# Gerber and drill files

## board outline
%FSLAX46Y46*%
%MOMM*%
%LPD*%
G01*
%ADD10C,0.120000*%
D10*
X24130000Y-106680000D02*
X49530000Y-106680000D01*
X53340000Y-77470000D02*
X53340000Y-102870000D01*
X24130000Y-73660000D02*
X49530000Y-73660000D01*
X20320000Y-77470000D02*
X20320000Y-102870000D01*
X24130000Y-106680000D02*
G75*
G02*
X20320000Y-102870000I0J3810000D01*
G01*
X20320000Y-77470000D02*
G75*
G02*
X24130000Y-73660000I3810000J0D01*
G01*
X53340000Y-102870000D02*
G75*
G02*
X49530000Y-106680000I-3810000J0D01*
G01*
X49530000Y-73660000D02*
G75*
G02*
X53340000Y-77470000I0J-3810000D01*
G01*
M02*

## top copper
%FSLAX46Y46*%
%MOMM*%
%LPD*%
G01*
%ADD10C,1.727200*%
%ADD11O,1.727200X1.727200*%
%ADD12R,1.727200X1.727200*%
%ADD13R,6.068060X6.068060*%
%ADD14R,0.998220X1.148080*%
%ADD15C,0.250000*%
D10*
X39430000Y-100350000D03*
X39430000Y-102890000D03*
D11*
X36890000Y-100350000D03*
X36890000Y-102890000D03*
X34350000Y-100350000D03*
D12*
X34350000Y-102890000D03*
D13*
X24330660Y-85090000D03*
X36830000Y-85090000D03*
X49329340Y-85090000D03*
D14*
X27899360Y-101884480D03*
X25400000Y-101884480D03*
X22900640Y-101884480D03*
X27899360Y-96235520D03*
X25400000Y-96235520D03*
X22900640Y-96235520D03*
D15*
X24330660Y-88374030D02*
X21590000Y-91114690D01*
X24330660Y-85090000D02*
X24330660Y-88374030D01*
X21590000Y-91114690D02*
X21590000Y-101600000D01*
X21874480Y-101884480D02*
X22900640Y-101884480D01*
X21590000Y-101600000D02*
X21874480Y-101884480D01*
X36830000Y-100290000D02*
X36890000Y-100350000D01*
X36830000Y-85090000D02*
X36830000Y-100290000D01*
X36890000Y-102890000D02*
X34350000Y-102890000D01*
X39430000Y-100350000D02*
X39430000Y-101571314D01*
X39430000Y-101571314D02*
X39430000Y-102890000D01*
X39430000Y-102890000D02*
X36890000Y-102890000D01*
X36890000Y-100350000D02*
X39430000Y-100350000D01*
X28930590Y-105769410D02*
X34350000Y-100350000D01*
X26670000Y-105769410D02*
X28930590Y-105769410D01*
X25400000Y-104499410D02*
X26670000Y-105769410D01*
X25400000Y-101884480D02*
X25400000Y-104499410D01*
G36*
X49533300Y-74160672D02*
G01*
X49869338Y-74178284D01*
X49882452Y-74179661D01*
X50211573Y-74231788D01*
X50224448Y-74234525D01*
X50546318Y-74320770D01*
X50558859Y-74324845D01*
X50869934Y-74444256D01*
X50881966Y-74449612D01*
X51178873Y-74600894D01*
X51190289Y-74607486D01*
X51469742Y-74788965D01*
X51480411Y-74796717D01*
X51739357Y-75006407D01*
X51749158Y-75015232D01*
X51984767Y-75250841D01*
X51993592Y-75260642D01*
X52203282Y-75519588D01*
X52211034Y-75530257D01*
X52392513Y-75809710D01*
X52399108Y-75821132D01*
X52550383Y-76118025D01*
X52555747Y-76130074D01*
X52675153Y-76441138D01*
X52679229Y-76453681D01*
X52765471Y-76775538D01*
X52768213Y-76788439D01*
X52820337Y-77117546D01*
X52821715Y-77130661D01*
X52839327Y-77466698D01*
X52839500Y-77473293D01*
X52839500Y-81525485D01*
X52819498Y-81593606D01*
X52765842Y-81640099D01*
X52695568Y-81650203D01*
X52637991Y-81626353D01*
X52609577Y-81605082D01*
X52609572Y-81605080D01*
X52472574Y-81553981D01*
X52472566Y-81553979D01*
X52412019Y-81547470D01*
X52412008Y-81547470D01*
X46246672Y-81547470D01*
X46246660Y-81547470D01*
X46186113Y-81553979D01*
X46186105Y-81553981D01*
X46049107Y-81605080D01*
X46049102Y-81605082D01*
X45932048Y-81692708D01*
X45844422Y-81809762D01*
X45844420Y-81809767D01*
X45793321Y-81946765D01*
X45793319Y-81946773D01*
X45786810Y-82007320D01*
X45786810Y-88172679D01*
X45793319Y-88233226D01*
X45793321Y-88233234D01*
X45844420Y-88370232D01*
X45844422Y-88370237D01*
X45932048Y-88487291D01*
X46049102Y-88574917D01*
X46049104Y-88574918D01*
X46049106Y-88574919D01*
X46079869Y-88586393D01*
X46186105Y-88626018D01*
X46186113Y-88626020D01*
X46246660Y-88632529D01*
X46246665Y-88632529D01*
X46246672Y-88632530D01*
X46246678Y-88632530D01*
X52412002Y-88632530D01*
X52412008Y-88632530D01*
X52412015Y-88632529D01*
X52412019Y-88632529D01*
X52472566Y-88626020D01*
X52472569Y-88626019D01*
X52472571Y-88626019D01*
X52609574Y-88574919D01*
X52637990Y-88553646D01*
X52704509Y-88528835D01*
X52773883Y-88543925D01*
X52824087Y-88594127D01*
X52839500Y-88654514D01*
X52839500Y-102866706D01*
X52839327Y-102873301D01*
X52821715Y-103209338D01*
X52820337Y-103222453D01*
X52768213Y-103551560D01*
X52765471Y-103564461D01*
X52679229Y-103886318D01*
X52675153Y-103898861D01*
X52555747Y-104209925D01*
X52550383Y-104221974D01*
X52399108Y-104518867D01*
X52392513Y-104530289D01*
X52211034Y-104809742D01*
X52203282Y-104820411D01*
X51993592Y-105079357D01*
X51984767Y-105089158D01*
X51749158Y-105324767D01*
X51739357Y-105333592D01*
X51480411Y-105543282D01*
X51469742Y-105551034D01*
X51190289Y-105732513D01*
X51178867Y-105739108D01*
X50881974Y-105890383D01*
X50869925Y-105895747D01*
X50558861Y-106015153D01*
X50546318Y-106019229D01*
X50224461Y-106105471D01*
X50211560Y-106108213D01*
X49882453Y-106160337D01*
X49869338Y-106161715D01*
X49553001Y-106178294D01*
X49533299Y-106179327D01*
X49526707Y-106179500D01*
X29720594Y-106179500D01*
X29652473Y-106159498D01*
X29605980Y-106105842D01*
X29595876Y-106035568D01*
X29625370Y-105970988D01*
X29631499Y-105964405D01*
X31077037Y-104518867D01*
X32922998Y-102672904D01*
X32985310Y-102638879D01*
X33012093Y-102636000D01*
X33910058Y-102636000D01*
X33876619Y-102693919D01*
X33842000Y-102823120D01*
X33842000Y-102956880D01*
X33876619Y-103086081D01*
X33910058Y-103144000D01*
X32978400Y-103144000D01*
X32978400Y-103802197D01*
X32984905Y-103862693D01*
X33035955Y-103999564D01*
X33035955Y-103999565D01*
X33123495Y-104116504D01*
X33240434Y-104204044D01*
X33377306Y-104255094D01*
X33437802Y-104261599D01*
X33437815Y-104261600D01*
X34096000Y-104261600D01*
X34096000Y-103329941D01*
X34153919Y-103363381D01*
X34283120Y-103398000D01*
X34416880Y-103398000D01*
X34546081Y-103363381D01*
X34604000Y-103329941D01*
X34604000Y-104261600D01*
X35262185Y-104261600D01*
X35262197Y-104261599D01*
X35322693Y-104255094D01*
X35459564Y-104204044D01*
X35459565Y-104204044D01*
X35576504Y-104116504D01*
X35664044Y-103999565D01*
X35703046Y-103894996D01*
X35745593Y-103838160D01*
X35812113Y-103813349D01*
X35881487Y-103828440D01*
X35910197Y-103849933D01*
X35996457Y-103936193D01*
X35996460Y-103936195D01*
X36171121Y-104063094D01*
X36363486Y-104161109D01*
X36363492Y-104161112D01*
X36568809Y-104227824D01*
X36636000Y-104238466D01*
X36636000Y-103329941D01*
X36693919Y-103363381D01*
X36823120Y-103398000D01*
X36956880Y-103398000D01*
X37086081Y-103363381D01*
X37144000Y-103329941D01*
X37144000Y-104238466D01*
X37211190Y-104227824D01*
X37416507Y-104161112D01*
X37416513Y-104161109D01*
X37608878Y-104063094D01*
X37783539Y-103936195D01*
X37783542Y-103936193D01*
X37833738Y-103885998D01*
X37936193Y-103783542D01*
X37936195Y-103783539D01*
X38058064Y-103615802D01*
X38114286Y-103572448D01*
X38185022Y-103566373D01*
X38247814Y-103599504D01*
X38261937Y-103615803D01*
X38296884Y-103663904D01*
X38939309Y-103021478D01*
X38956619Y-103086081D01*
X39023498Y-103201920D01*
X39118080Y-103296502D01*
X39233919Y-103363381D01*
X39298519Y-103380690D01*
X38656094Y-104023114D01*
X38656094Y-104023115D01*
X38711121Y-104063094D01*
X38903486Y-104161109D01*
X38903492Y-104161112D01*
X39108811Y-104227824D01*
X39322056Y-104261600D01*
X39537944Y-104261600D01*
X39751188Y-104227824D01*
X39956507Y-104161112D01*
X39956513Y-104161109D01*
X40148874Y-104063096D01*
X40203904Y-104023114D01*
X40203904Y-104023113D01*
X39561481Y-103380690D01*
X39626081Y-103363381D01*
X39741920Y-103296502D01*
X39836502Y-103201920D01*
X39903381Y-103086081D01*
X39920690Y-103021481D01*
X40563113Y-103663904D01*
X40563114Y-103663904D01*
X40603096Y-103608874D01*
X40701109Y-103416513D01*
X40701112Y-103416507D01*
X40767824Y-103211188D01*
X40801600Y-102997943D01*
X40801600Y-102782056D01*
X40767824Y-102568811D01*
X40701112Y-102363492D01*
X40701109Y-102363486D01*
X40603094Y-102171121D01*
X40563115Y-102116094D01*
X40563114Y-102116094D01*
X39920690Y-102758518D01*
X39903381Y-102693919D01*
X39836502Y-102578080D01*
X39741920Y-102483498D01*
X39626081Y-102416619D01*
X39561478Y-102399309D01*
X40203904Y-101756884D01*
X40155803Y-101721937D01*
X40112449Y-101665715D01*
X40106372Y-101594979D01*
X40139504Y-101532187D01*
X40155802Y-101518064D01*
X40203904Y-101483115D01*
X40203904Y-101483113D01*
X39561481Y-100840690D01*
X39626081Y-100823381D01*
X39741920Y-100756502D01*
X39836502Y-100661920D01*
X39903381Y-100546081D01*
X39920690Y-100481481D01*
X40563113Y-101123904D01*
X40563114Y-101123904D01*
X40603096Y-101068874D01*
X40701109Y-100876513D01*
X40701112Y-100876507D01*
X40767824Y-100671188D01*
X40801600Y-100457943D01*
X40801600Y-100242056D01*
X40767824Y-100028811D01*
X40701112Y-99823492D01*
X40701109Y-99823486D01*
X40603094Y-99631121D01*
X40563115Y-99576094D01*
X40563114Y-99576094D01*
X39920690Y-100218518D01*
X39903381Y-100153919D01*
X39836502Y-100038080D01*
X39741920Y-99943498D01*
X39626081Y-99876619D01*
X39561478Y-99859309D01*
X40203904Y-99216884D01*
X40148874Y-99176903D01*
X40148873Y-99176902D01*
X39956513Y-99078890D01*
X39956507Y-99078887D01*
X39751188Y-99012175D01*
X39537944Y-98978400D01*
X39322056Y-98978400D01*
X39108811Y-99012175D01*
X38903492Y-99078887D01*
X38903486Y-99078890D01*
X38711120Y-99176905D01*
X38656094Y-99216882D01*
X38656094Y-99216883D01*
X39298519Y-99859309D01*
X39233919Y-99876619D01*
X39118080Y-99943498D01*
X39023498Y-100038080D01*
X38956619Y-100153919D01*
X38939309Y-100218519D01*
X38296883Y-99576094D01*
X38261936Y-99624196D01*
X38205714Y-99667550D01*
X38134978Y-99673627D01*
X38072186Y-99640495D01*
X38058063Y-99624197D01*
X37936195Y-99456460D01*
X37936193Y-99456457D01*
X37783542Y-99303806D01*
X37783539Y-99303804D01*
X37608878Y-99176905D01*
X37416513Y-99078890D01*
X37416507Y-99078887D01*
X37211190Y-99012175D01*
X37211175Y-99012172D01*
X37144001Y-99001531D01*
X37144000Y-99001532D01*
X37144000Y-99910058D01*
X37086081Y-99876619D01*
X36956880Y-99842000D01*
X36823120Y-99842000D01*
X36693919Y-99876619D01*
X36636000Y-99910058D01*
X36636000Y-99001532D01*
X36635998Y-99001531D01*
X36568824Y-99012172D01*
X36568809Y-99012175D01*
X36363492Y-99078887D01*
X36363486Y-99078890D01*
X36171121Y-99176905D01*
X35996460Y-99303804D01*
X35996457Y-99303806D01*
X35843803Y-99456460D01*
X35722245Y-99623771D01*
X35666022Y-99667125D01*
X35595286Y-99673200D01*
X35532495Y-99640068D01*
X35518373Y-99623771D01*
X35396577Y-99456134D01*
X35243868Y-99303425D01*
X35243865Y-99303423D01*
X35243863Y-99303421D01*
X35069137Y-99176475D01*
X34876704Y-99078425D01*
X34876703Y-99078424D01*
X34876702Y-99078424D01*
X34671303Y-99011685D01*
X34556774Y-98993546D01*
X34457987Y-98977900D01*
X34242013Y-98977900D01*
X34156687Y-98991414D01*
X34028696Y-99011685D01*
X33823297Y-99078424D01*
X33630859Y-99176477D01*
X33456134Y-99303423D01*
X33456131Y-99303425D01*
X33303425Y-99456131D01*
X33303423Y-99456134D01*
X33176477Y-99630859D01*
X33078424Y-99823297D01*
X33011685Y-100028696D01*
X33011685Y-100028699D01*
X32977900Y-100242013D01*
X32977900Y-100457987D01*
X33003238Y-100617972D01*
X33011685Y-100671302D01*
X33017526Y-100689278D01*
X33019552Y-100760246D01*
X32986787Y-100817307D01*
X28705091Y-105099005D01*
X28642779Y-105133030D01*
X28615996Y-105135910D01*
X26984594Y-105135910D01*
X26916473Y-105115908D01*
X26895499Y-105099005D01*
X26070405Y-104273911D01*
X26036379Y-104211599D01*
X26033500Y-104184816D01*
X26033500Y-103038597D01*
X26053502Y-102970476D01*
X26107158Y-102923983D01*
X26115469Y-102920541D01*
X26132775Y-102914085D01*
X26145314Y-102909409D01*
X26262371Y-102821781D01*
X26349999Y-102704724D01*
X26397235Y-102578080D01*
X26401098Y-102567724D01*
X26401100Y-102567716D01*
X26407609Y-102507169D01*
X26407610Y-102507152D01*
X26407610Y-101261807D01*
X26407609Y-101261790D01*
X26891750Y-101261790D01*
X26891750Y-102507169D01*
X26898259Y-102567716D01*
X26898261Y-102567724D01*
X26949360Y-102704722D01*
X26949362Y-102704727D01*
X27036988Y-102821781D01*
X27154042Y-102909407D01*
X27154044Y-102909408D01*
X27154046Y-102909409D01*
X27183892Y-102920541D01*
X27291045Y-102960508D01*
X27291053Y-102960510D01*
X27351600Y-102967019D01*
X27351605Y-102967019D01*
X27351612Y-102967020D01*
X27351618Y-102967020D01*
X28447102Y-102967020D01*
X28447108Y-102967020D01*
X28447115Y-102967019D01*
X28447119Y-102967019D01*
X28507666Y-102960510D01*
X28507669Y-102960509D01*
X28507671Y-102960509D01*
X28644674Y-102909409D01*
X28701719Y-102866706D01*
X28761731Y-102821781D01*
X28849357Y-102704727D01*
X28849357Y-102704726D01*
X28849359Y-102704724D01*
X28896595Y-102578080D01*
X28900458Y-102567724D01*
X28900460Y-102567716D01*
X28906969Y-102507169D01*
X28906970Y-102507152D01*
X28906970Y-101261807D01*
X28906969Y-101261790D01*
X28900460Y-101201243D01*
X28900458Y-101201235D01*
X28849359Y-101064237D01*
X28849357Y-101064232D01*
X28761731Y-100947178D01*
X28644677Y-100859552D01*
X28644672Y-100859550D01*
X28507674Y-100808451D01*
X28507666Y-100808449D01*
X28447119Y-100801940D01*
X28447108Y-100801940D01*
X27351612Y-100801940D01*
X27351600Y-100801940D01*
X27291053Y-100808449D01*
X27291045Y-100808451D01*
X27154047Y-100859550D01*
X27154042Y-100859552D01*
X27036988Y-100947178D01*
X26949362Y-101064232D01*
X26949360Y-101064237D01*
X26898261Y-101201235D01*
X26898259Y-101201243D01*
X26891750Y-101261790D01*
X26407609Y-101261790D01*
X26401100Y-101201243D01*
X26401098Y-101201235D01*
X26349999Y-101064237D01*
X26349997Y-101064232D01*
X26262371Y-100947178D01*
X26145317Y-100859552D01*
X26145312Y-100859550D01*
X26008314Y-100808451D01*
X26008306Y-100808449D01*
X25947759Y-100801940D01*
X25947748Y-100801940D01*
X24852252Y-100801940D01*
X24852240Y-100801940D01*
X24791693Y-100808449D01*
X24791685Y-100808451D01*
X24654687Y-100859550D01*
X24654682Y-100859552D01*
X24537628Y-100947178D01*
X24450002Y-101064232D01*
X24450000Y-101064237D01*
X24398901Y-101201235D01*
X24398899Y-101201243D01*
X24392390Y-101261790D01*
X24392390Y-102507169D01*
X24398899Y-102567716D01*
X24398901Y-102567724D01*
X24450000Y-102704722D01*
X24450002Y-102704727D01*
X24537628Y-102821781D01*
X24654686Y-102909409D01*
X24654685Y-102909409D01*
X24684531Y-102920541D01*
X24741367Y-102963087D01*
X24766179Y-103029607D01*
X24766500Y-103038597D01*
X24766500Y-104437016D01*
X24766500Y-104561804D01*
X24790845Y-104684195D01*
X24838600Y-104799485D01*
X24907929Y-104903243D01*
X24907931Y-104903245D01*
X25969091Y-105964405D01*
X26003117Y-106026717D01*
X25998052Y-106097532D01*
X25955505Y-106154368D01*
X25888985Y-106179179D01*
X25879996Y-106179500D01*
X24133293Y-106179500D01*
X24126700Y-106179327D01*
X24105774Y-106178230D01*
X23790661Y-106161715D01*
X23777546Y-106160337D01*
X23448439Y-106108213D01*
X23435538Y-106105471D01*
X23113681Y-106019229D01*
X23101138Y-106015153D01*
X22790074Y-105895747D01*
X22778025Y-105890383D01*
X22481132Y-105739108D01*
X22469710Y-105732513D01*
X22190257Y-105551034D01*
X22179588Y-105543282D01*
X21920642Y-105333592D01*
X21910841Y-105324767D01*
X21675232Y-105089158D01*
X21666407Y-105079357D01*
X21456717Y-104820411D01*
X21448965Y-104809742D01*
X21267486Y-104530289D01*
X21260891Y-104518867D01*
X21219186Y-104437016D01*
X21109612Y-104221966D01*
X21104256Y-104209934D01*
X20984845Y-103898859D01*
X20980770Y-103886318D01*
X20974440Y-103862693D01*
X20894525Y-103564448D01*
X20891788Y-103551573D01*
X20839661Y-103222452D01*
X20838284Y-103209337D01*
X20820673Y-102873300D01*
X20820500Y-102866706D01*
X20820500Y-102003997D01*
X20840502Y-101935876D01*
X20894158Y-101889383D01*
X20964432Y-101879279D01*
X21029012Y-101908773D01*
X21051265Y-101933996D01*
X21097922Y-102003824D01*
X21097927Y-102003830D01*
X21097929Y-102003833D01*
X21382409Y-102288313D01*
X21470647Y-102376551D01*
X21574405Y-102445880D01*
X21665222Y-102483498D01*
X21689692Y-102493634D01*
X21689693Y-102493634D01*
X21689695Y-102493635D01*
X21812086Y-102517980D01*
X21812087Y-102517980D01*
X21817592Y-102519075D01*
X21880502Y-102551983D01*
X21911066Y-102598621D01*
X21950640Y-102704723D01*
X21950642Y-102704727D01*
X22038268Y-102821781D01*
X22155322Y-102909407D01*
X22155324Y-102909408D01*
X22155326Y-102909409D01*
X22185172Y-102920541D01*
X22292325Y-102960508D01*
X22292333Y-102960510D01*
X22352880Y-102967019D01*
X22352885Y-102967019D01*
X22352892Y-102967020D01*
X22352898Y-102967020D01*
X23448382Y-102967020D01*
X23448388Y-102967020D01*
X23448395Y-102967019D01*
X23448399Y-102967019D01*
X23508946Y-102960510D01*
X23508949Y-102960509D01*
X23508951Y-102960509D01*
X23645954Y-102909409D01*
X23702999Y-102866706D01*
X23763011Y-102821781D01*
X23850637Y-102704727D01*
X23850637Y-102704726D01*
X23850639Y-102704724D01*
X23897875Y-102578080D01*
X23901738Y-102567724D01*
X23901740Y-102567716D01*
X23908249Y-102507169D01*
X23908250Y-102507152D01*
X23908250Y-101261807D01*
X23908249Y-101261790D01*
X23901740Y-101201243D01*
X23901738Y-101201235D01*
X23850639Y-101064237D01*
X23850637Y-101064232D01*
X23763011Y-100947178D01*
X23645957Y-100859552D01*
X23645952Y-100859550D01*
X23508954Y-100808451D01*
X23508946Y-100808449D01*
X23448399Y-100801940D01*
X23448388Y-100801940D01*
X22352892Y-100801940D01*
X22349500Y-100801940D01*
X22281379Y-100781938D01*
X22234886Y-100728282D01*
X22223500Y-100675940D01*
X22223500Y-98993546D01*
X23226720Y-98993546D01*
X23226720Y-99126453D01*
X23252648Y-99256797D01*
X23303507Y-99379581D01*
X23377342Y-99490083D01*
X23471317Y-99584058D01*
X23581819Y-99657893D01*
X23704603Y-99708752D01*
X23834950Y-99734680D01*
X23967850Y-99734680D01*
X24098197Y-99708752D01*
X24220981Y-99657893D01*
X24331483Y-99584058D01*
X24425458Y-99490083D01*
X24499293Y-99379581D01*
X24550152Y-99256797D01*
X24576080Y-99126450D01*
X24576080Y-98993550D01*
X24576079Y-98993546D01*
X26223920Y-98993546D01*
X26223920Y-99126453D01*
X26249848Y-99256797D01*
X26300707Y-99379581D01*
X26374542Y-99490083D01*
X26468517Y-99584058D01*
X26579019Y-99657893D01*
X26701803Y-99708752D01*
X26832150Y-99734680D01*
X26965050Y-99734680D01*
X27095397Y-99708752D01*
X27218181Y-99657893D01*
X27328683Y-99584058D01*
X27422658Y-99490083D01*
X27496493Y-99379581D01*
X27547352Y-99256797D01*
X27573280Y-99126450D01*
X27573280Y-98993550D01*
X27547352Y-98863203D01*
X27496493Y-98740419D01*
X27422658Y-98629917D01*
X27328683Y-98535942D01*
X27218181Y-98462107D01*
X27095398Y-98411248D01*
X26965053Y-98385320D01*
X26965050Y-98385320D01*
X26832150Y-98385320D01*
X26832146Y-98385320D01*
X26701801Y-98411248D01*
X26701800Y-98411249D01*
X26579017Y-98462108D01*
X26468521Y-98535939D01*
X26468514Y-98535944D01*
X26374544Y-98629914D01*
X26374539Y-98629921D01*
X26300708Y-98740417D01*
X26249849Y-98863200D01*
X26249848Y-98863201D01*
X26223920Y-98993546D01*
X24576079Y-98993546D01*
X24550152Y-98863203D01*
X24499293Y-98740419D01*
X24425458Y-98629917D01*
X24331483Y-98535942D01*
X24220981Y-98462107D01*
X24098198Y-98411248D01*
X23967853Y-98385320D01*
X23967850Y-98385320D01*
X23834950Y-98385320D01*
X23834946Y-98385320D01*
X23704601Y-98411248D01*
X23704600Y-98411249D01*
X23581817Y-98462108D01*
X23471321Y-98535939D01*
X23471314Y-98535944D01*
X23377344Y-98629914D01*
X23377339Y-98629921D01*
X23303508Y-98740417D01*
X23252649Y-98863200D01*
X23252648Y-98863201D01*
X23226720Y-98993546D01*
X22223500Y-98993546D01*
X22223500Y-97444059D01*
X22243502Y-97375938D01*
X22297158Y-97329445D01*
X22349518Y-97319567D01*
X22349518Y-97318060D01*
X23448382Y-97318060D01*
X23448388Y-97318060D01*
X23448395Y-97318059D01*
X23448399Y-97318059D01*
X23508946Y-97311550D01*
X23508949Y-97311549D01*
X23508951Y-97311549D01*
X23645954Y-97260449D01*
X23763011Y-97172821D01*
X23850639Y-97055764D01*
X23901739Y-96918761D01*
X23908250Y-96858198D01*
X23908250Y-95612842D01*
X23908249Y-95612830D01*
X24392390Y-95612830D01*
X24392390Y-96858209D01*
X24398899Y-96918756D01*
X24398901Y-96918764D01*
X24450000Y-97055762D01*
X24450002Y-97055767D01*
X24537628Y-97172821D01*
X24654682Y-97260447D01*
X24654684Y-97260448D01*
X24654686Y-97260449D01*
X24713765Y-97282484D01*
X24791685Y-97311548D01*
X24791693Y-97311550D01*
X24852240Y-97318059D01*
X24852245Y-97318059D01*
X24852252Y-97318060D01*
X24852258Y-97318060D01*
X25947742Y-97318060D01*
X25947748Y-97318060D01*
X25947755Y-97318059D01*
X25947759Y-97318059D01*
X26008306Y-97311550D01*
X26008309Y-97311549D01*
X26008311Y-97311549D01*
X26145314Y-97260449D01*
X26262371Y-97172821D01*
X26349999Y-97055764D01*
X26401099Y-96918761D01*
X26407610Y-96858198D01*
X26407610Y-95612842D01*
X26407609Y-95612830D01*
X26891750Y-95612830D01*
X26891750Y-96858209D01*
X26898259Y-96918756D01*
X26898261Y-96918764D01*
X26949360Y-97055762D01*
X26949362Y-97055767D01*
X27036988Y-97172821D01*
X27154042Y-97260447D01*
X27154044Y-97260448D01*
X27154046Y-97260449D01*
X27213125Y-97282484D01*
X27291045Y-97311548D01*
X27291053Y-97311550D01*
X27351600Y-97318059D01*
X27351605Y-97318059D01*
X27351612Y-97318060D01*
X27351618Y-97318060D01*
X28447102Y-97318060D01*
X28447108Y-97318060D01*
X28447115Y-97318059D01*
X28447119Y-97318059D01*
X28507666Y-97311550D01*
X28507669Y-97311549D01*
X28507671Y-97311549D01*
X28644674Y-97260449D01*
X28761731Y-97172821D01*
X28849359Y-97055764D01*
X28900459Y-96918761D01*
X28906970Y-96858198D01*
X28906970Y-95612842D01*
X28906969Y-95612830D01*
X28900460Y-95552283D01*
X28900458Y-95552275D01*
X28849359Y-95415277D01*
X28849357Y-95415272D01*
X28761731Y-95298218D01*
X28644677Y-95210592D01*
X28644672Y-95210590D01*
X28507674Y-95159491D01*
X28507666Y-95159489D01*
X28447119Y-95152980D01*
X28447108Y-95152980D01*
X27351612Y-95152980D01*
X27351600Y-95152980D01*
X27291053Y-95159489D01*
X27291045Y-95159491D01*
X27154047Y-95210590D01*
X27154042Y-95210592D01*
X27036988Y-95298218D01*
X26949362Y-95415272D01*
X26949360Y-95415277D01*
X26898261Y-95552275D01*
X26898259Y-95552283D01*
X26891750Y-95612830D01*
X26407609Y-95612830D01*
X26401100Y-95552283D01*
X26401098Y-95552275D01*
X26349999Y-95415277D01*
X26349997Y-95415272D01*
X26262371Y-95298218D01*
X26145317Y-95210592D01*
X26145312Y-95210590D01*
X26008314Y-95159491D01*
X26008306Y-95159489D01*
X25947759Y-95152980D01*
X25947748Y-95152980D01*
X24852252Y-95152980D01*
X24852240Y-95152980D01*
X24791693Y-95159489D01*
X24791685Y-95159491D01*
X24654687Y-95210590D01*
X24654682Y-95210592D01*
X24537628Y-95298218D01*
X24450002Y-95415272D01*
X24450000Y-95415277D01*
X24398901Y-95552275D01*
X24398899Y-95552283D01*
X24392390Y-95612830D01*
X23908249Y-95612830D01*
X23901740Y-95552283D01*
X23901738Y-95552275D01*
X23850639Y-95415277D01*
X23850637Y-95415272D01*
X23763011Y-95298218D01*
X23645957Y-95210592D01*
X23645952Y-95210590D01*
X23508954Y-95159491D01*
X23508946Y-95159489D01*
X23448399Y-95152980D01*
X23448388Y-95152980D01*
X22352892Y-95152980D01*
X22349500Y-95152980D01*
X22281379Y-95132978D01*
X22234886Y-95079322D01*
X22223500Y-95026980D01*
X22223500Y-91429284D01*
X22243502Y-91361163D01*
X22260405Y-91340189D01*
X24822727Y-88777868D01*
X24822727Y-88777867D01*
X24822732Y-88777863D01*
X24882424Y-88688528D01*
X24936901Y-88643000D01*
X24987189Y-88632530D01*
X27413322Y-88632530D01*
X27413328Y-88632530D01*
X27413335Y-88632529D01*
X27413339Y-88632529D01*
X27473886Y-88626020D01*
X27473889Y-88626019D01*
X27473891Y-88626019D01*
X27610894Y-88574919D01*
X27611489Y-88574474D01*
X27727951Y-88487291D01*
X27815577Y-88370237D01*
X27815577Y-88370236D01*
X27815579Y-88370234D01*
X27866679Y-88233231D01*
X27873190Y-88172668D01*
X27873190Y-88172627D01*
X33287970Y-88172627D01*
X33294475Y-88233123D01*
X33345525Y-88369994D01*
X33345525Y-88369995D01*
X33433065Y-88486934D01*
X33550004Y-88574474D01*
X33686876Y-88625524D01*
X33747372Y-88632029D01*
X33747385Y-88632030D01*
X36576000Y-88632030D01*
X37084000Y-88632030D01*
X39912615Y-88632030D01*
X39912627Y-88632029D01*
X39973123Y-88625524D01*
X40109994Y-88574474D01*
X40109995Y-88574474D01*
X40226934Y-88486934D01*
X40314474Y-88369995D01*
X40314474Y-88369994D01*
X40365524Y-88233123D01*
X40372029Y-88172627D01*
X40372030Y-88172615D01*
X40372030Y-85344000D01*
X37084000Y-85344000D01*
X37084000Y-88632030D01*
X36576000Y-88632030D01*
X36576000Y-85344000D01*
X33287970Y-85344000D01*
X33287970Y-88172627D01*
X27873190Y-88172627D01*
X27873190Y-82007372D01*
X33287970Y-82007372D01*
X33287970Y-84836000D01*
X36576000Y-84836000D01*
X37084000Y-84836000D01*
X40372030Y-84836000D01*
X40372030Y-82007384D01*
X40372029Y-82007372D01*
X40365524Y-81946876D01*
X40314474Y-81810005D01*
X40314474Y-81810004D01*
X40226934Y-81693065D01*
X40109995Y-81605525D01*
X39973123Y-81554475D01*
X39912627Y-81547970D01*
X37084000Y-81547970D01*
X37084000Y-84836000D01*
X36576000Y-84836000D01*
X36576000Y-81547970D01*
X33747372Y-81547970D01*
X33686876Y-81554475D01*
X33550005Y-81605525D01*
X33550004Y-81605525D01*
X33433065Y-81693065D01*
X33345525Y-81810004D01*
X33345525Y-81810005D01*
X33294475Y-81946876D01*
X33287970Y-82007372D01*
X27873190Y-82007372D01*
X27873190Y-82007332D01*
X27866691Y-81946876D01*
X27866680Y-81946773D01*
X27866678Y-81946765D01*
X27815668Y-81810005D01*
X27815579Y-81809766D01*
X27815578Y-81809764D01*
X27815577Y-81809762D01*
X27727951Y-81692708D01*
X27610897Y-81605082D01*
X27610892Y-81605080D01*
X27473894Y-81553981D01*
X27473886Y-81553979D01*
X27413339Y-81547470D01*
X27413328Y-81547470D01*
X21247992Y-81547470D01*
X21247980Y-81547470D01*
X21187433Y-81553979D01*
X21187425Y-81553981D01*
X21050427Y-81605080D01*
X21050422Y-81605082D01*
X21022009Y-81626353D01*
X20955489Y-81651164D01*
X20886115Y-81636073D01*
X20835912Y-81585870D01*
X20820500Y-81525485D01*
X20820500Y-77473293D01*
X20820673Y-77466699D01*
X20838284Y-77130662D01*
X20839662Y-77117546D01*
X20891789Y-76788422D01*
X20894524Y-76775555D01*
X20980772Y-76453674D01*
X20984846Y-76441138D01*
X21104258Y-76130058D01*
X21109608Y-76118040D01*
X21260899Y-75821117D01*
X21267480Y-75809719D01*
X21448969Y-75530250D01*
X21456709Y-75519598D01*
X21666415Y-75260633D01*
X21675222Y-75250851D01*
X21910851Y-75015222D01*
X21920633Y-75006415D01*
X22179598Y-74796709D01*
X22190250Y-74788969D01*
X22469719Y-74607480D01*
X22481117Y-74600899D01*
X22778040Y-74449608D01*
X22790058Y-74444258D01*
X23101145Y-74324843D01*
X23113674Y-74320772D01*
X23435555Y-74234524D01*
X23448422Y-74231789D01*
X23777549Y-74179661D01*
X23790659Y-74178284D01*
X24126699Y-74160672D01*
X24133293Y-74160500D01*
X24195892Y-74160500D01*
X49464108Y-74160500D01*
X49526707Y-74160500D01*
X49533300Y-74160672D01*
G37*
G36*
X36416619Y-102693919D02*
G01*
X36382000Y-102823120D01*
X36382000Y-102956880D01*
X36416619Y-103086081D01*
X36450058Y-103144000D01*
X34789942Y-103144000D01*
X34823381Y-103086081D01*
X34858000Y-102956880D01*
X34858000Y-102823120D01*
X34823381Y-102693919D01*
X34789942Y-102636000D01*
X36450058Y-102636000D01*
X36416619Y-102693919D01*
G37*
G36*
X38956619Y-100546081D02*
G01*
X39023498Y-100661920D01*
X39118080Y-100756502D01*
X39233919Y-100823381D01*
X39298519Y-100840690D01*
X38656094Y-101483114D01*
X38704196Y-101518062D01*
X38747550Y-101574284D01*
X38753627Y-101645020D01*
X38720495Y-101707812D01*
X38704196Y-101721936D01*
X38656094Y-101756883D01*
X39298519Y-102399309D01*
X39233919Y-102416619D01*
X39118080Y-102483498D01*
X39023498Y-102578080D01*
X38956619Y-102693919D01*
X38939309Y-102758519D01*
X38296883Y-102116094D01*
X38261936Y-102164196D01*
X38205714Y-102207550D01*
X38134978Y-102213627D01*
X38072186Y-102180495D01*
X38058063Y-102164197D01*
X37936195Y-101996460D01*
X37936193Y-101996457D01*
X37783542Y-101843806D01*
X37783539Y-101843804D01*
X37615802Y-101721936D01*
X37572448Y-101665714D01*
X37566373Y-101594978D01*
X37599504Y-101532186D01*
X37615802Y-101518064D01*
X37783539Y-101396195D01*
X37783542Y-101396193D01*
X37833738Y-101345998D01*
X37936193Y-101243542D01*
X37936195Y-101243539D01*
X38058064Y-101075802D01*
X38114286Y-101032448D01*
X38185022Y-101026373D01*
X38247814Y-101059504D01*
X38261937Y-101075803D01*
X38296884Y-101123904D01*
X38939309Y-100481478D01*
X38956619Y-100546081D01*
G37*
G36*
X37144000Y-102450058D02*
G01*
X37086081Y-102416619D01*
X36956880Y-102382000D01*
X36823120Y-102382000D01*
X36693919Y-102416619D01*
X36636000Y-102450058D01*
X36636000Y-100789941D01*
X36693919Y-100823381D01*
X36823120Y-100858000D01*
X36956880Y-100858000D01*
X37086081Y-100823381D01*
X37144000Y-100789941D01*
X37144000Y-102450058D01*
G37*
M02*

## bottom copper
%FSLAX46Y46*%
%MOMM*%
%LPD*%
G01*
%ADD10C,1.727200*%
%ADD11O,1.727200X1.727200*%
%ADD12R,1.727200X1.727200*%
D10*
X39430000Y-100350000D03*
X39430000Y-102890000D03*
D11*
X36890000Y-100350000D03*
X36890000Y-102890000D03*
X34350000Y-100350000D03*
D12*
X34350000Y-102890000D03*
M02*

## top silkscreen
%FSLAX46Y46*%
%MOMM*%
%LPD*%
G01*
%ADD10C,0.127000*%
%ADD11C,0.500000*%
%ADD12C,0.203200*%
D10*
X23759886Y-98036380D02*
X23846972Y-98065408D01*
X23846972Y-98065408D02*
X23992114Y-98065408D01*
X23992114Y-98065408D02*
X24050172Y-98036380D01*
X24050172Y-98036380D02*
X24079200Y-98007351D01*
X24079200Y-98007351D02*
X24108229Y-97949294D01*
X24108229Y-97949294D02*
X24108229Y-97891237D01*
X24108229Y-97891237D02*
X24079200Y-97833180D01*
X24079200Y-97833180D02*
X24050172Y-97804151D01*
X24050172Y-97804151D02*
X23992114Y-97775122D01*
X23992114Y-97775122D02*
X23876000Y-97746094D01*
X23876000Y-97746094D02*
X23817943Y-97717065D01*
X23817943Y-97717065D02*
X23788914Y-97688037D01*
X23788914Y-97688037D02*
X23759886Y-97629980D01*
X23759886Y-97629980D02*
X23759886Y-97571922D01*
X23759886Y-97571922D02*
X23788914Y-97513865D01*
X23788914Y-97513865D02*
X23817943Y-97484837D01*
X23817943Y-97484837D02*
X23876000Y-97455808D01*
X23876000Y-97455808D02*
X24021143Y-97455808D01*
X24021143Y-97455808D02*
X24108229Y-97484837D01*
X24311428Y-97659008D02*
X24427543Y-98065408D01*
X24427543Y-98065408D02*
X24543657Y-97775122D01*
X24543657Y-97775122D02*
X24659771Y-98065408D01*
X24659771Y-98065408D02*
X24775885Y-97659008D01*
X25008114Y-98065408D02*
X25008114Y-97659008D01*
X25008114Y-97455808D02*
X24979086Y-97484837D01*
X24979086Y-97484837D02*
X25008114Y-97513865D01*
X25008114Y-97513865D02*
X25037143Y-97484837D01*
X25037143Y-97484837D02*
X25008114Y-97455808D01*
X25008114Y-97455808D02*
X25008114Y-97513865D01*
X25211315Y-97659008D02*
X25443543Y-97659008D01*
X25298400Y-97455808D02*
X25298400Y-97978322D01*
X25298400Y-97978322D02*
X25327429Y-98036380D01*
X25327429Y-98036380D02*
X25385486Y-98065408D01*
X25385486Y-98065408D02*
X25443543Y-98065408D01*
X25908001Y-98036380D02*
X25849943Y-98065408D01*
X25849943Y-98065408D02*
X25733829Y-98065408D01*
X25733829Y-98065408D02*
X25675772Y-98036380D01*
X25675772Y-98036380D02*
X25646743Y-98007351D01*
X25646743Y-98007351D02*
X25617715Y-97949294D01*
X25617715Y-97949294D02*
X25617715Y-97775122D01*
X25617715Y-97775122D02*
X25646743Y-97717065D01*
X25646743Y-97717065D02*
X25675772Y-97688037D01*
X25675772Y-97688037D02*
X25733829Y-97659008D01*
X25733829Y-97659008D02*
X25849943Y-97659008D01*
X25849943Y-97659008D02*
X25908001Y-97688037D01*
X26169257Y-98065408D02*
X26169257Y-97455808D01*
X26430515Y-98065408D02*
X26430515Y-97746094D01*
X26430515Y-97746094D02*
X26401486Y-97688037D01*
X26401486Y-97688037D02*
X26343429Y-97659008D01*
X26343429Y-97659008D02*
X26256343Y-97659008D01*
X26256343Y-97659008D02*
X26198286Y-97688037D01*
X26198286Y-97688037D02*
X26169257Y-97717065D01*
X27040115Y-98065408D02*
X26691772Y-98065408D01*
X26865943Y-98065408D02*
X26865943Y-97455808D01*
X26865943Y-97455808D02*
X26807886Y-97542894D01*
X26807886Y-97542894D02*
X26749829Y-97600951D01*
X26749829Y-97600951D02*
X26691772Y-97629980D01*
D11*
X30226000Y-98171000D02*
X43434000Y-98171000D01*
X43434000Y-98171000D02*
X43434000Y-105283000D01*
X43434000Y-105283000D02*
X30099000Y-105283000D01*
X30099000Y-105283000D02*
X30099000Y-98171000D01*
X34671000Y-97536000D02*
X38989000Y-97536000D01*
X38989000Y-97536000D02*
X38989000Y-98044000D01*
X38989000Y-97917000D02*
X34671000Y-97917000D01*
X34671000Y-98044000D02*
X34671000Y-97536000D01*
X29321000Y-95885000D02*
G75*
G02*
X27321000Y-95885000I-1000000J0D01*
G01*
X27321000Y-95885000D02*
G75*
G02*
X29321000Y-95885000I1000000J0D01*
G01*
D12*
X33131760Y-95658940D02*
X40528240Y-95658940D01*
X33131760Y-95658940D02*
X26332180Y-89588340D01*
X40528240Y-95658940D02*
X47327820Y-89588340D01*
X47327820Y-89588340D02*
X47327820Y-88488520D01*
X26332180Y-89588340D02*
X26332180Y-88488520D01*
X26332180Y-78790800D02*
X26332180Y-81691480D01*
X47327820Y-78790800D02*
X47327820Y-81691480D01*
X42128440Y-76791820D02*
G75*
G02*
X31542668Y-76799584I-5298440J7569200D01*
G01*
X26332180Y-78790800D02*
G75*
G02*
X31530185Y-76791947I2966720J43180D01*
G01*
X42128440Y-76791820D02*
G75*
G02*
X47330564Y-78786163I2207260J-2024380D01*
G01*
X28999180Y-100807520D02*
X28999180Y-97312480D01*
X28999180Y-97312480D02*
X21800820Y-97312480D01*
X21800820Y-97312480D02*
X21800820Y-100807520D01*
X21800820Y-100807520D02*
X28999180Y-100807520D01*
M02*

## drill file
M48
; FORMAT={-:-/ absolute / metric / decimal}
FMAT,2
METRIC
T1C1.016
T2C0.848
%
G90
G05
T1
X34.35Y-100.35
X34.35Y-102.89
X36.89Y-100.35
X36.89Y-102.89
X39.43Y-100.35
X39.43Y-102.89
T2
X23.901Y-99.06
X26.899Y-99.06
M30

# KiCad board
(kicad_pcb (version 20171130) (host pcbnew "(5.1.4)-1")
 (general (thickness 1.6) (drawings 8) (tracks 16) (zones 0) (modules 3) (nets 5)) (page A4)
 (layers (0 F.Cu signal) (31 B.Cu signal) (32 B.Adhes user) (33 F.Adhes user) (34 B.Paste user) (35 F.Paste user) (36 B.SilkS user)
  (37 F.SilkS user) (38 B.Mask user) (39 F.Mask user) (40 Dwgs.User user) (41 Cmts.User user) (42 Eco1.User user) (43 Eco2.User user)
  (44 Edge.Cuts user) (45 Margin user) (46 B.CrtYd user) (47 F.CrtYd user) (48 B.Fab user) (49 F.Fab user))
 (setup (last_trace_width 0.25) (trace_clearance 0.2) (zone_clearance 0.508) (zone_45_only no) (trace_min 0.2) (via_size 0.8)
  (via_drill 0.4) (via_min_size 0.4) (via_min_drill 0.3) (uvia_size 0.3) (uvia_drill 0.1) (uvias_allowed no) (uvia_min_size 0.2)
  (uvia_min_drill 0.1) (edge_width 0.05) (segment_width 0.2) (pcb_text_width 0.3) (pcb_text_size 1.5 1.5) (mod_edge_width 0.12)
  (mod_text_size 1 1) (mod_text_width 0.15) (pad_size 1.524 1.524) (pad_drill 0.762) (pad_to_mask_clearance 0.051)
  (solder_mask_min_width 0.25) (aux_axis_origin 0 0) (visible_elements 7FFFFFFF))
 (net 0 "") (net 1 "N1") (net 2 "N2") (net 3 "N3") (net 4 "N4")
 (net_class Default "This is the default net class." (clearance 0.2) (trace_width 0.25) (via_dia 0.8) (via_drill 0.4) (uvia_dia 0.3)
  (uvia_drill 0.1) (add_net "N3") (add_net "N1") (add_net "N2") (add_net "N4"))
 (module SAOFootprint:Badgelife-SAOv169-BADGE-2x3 (layer F.Cu) (at 36.83 101.6)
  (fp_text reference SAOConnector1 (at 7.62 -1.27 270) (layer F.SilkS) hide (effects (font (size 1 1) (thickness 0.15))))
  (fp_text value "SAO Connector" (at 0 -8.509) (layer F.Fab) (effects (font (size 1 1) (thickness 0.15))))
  (fp_line (start -6.604 -3.429) (end 6.604 -3.429) (layer F.SilkS) (width 0.5))
  (fp_line (start 6.604 -3.429) (end 6.604 3.683) (layer F.SilkS) (width 0.5))
  (fp_line (start 6.604 3.683) (end -6.731 3.683) (layer F.SilkS) (width 0.5))
  (fp_line (start -6.731 3.683) (end -6.731 -3.429) (layer F.SilkS) (width 0.5))
  (fp_line (start -2.159 -4.064) (end 2.159 -4.064) (layer F.SilkS) (width 0.5))
  (fp_line (start 2.159 -4.064) (end 2.159 -3.556) (layer F.SilkS) (width 0.5))
  (fp_line (start 2.159 -3.683) (end -2.159 -3.683) (layer F.SilkS) (width 0.5))
  (fp_line (start -2.159 -3.556) (end -2.159 -4.064) (layer F.SilkS) (width 0.5))
  (fp_circle (center -8.509 -5.715) (end -7.509 -5.715) (layer F.SilkS) (width 0.5))
  (pad 5 thru_hole circle (at 2.6 -1.25 270) (size 1.7272 1.7272) (drill 1.016) (layers *.Cu *.Mask) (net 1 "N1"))
  (pad 6 thru_hole circle (at 2.6 1.29 270) (size 1.7272 1.7272) (drill 1.016) (layers *.Cu *.Mask) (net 1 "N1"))
  (pad 3 thru_hole oval (at 0.06 -1.25 270) (size 1.7272 1.7272) (drill 1.016) (layers *.Cu *.Mask) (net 1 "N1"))
  (pad 4 thru_hole oval (at 0.06 1.29 270) (size 1.7272 1.7272) (drill 1.016) (layers *.Cu *.Mask) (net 1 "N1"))
  (pad 1 thru_hole oval (at -2.48 -1.25 270) (size 1.7272 1.7272) (drill 1.016) (layers *.Cu *.Mask) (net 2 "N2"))
  (pad 2 thru_hole rect (at -2.48 1.29 270) (size 1.7272 1.7272) (drill 1.016) (layers *.Cu *.Mask) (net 1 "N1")))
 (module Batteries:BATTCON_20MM (layer F.Cu) (at 36.83 85.09)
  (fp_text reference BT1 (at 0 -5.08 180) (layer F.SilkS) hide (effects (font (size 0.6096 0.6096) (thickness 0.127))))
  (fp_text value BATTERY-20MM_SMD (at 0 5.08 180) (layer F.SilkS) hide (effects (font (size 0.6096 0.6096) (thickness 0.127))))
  (fp_line (start -3.69824 10.56894) (end 3.69824 10.56894) (layer F.SilkS) (width 0.2032))
  (fp_line (start -3.69824 10.56894) (end -10.49782 4.49834) (layer F.SilkS) (width 0.2032))
  (fp_line (start 3.69824 10.56894) (end 10.49782 4.49834) (layer F.SilkS) (width 0.2032))
  (fp_line (start 10.49782 4.49834) (end 10.49782 3.39852) (layer F.SilkS) (width 0.2032))
  (fp_line (start -10.49782 4.49834) (end -10.49782 3.39852) (layer F.SilkS) (width 0.2032))
  (fp_line (start -10.49782 -6.2992) (end -10.49782 -3.39852) (layer F.SilkS) (width 0.2032))
  (fp_line (start 10.49782 -6.2992) (end 10.49782 -3.39852) (layer F.SilkS) (width 0.2032))
  (fp_arc (start 0 -15.86738) (end 5.29844 -8.29818) (angle 69.9) (layer F.SilkS) (width 0.2032))
  (fp_arc (start -7.5311 -6.34238) (end -10.49782 -6.2992) (angle 139.6) (layer F.SilkS) (width 0.2032))
  (fp_arc (start 7.5057 -6.2738) (end 5.29844 -8.29818) (angle 136.9) (layer F.SilkS) (width 0.2032))
  (pad 1 smd rect (at -12.49934 0) (size 6.06806 6.06806) (layers F.Cu F.Paste F.Mask) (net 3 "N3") (solder_mask_margin 0.1016))
  (pad 2 smd rect (at 0 0) (size 6.06806 6.06806) (layers F.Cu F.Paste F.Mask) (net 1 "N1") (solder_mask_margin 0.1016))
  (pad 3 smd rect (at 12.49934 0) (size 6.06806 6.06806) (layers F.Cu F.Paste F.Mask) (solder_mask_margin 0.1016)))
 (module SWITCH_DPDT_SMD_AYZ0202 (layer F.Cu) (at 25.4 99.06 180)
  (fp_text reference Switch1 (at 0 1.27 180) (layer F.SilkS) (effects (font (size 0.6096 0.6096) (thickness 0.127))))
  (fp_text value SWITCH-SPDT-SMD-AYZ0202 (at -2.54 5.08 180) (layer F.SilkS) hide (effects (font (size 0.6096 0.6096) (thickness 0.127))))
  (fp_line (start -3.59918 -1.74752) (end -3.59918 1.74752) (layer F.SilkS) (width 0.2032))
  (fp_line (start -3.59918 1.74752) (end 3.59918 1.74752) (layer F.SilkS) (width 0.2032))
  (fp_line (start 3.59918 1.74752) (end 3.59918 -1.74752) (layer F.SilkS) (width 0.2032))
  (fp_line (start 3.59918 -1.74752) (end -3.59918 -1.74752) (layer F.SilkS) (width 0.2032))
  (pad 1 smd rect (at -2.49936 -2.82448 180) (size 0.99822 1.14808) (layers F.Cu F.Paste F.Mask) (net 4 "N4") (solder_mask_margin 0.1016))
  (pad 2 smd rect (at 0 -2.82448 180) (size 0.99822 1.14808) (layers F.Cu F.Paste F.Mask) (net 2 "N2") (solder_mask_margin 0.1016))
  (pad 3 smd rect (at 2.49936 -2.82448 180) (size 0.99822 1.14808) (layers F.Cu F.Paste F.Mask) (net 3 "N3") (solder_mask_margin 0.1016))
  (pad 4 smd rect (at -2.49936 2.82448 180) (size 0.99822 1.14808) (layers F.Cu F.Paste F.Mask) (solder_mask_margin 0.1016))
  (pad 5 smd rect (at 0 2.82448 180) (size 0.99822 1.14808) (layers F.Cu F.Paste F.Mask) (solder_mask_margin 0.1016))
  (pad 6 smd rect (at 2.49936 2.82448 180) (size 0.99822 1.14808) (layers F.Cu F.Paste F.Mask) (solder_mask_margin 0.1016))
  (pad "" np_thru_hole circle (at 1.4986 0 180) (size 0.84836 0.84836) (drill 0.84836) (layers *.Cu *.Mask) (solder_mask_margin 0.1016))
  (pad "" np_thru_hole circle (at -1.4986 0 180) (size 0.84836 0.84836) (drill 0.84836) (layers *.Cu *.Mask) (solder_mask_margin 0.1016)))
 (gr_line (start 24.13 106.68) (end 49.53 106.68) (layer Edge.Cuts) (width 0.12))
 (gr_line (start 53.34 77.47) (end 53.34 102.87) (layer Edge.Cuts) (width 0.12))
 (gr_line (start 24.13 73.66) (end 49.53 73.66) (layer Edge.Cuts) (width 0.12))
 (gr_line (start 20.32 77.47) (end 20.32 102.87) (layer Edge.Cuts) (width 0.12))
 (gr_arc (start 24.13 102.87) (end 24.13 106.68) (angle 90) (layer Edge.Cuts) (width 0.12))
 (gr_arc (start 24.13 77.47) (end 24.13 73.66) (angle -90) (layer Edge.Cuts) (width 0.12))
 (gr_arc (start 49.53 102.87) (end 53.34 102.87) (angle 90) (layer Edge.Cuts) (width 0.12))
 (gr_arc (start 49.53 77.47) (end 53.34 77.47) (angle -90) (layer Edge.Cuts) (width 0.12))
 (segment (start 24.33066 88.37403) (end 21.59 91.11469) (width 0.25) (layer F.Cu) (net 3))
 (segment (start 24.33066 85.09) (end 24.33066 88.37403) (width 0.25) (layer F.Cu) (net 3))
 (segment (start 21.59 91.11469) (end 21.59 101.6) (width 0.25) (layer F.Cu) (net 3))
 (segment (start 21.87448 101.88448) (end 22.90064 101.88448) (width 0.25) (layer F.Cu) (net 3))
 (segment (start 21.59 101.6) (end 21.87448 101.88448) (width 0.25) (layer F.Cu) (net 3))
 (segment (start 36.83 100.29) (end 36.89 100.35) (width 0.25) (layer F.Cu) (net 1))
 (segment (start 36.83 85.09) (end 36.83 100.29) (width 0.25) (layer F.Cu) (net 1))
 (segment (start 36.89 102.89) (end 34.35 102.89) (width 0.25) (layer F.Cu) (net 1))
 (segment (start 39.43 100.35) (end 39.43 101.571314) (width 0.25) (layer F.Cu) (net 1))
 (segment (start 39.43 101.571314) (end 39.43 102.89) (width 0.25) (layer F.Cu) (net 1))
 (segment (start 39.43 102.89) (end 36.89 102.89) (width 0.25) (layer F.Cu) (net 1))
 (segment (start 36.89 100.35) (end 39.43 100.35) (width 0.25) (layer F.Cu) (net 1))
 (segment (start 28.93059 105.76941) (end 34.35 100.35) (width 0.25) (layer F.Cu) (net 2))
 (segment (start 26.67 105.76941) (end 28.93059 105.76941) (width 0.25) (layer F.Cu) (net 2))
 (segment (start 25.4 104.49941) (end 26.67 105.76941) (width 0.25) (layer F.Cu) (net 2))
 (segment (start 25.4 101.88448) (end 25.4 104.49941) (width 0.25) (layer F.Cu) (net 2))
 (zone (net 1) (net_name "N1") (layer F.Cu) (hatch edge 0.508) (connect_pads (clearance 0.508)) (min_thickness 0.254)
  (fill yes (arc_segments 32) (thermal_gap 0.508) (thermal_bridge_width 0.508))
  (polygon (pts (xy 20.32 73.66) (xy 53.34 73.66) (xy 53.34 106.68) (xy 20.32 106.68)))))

